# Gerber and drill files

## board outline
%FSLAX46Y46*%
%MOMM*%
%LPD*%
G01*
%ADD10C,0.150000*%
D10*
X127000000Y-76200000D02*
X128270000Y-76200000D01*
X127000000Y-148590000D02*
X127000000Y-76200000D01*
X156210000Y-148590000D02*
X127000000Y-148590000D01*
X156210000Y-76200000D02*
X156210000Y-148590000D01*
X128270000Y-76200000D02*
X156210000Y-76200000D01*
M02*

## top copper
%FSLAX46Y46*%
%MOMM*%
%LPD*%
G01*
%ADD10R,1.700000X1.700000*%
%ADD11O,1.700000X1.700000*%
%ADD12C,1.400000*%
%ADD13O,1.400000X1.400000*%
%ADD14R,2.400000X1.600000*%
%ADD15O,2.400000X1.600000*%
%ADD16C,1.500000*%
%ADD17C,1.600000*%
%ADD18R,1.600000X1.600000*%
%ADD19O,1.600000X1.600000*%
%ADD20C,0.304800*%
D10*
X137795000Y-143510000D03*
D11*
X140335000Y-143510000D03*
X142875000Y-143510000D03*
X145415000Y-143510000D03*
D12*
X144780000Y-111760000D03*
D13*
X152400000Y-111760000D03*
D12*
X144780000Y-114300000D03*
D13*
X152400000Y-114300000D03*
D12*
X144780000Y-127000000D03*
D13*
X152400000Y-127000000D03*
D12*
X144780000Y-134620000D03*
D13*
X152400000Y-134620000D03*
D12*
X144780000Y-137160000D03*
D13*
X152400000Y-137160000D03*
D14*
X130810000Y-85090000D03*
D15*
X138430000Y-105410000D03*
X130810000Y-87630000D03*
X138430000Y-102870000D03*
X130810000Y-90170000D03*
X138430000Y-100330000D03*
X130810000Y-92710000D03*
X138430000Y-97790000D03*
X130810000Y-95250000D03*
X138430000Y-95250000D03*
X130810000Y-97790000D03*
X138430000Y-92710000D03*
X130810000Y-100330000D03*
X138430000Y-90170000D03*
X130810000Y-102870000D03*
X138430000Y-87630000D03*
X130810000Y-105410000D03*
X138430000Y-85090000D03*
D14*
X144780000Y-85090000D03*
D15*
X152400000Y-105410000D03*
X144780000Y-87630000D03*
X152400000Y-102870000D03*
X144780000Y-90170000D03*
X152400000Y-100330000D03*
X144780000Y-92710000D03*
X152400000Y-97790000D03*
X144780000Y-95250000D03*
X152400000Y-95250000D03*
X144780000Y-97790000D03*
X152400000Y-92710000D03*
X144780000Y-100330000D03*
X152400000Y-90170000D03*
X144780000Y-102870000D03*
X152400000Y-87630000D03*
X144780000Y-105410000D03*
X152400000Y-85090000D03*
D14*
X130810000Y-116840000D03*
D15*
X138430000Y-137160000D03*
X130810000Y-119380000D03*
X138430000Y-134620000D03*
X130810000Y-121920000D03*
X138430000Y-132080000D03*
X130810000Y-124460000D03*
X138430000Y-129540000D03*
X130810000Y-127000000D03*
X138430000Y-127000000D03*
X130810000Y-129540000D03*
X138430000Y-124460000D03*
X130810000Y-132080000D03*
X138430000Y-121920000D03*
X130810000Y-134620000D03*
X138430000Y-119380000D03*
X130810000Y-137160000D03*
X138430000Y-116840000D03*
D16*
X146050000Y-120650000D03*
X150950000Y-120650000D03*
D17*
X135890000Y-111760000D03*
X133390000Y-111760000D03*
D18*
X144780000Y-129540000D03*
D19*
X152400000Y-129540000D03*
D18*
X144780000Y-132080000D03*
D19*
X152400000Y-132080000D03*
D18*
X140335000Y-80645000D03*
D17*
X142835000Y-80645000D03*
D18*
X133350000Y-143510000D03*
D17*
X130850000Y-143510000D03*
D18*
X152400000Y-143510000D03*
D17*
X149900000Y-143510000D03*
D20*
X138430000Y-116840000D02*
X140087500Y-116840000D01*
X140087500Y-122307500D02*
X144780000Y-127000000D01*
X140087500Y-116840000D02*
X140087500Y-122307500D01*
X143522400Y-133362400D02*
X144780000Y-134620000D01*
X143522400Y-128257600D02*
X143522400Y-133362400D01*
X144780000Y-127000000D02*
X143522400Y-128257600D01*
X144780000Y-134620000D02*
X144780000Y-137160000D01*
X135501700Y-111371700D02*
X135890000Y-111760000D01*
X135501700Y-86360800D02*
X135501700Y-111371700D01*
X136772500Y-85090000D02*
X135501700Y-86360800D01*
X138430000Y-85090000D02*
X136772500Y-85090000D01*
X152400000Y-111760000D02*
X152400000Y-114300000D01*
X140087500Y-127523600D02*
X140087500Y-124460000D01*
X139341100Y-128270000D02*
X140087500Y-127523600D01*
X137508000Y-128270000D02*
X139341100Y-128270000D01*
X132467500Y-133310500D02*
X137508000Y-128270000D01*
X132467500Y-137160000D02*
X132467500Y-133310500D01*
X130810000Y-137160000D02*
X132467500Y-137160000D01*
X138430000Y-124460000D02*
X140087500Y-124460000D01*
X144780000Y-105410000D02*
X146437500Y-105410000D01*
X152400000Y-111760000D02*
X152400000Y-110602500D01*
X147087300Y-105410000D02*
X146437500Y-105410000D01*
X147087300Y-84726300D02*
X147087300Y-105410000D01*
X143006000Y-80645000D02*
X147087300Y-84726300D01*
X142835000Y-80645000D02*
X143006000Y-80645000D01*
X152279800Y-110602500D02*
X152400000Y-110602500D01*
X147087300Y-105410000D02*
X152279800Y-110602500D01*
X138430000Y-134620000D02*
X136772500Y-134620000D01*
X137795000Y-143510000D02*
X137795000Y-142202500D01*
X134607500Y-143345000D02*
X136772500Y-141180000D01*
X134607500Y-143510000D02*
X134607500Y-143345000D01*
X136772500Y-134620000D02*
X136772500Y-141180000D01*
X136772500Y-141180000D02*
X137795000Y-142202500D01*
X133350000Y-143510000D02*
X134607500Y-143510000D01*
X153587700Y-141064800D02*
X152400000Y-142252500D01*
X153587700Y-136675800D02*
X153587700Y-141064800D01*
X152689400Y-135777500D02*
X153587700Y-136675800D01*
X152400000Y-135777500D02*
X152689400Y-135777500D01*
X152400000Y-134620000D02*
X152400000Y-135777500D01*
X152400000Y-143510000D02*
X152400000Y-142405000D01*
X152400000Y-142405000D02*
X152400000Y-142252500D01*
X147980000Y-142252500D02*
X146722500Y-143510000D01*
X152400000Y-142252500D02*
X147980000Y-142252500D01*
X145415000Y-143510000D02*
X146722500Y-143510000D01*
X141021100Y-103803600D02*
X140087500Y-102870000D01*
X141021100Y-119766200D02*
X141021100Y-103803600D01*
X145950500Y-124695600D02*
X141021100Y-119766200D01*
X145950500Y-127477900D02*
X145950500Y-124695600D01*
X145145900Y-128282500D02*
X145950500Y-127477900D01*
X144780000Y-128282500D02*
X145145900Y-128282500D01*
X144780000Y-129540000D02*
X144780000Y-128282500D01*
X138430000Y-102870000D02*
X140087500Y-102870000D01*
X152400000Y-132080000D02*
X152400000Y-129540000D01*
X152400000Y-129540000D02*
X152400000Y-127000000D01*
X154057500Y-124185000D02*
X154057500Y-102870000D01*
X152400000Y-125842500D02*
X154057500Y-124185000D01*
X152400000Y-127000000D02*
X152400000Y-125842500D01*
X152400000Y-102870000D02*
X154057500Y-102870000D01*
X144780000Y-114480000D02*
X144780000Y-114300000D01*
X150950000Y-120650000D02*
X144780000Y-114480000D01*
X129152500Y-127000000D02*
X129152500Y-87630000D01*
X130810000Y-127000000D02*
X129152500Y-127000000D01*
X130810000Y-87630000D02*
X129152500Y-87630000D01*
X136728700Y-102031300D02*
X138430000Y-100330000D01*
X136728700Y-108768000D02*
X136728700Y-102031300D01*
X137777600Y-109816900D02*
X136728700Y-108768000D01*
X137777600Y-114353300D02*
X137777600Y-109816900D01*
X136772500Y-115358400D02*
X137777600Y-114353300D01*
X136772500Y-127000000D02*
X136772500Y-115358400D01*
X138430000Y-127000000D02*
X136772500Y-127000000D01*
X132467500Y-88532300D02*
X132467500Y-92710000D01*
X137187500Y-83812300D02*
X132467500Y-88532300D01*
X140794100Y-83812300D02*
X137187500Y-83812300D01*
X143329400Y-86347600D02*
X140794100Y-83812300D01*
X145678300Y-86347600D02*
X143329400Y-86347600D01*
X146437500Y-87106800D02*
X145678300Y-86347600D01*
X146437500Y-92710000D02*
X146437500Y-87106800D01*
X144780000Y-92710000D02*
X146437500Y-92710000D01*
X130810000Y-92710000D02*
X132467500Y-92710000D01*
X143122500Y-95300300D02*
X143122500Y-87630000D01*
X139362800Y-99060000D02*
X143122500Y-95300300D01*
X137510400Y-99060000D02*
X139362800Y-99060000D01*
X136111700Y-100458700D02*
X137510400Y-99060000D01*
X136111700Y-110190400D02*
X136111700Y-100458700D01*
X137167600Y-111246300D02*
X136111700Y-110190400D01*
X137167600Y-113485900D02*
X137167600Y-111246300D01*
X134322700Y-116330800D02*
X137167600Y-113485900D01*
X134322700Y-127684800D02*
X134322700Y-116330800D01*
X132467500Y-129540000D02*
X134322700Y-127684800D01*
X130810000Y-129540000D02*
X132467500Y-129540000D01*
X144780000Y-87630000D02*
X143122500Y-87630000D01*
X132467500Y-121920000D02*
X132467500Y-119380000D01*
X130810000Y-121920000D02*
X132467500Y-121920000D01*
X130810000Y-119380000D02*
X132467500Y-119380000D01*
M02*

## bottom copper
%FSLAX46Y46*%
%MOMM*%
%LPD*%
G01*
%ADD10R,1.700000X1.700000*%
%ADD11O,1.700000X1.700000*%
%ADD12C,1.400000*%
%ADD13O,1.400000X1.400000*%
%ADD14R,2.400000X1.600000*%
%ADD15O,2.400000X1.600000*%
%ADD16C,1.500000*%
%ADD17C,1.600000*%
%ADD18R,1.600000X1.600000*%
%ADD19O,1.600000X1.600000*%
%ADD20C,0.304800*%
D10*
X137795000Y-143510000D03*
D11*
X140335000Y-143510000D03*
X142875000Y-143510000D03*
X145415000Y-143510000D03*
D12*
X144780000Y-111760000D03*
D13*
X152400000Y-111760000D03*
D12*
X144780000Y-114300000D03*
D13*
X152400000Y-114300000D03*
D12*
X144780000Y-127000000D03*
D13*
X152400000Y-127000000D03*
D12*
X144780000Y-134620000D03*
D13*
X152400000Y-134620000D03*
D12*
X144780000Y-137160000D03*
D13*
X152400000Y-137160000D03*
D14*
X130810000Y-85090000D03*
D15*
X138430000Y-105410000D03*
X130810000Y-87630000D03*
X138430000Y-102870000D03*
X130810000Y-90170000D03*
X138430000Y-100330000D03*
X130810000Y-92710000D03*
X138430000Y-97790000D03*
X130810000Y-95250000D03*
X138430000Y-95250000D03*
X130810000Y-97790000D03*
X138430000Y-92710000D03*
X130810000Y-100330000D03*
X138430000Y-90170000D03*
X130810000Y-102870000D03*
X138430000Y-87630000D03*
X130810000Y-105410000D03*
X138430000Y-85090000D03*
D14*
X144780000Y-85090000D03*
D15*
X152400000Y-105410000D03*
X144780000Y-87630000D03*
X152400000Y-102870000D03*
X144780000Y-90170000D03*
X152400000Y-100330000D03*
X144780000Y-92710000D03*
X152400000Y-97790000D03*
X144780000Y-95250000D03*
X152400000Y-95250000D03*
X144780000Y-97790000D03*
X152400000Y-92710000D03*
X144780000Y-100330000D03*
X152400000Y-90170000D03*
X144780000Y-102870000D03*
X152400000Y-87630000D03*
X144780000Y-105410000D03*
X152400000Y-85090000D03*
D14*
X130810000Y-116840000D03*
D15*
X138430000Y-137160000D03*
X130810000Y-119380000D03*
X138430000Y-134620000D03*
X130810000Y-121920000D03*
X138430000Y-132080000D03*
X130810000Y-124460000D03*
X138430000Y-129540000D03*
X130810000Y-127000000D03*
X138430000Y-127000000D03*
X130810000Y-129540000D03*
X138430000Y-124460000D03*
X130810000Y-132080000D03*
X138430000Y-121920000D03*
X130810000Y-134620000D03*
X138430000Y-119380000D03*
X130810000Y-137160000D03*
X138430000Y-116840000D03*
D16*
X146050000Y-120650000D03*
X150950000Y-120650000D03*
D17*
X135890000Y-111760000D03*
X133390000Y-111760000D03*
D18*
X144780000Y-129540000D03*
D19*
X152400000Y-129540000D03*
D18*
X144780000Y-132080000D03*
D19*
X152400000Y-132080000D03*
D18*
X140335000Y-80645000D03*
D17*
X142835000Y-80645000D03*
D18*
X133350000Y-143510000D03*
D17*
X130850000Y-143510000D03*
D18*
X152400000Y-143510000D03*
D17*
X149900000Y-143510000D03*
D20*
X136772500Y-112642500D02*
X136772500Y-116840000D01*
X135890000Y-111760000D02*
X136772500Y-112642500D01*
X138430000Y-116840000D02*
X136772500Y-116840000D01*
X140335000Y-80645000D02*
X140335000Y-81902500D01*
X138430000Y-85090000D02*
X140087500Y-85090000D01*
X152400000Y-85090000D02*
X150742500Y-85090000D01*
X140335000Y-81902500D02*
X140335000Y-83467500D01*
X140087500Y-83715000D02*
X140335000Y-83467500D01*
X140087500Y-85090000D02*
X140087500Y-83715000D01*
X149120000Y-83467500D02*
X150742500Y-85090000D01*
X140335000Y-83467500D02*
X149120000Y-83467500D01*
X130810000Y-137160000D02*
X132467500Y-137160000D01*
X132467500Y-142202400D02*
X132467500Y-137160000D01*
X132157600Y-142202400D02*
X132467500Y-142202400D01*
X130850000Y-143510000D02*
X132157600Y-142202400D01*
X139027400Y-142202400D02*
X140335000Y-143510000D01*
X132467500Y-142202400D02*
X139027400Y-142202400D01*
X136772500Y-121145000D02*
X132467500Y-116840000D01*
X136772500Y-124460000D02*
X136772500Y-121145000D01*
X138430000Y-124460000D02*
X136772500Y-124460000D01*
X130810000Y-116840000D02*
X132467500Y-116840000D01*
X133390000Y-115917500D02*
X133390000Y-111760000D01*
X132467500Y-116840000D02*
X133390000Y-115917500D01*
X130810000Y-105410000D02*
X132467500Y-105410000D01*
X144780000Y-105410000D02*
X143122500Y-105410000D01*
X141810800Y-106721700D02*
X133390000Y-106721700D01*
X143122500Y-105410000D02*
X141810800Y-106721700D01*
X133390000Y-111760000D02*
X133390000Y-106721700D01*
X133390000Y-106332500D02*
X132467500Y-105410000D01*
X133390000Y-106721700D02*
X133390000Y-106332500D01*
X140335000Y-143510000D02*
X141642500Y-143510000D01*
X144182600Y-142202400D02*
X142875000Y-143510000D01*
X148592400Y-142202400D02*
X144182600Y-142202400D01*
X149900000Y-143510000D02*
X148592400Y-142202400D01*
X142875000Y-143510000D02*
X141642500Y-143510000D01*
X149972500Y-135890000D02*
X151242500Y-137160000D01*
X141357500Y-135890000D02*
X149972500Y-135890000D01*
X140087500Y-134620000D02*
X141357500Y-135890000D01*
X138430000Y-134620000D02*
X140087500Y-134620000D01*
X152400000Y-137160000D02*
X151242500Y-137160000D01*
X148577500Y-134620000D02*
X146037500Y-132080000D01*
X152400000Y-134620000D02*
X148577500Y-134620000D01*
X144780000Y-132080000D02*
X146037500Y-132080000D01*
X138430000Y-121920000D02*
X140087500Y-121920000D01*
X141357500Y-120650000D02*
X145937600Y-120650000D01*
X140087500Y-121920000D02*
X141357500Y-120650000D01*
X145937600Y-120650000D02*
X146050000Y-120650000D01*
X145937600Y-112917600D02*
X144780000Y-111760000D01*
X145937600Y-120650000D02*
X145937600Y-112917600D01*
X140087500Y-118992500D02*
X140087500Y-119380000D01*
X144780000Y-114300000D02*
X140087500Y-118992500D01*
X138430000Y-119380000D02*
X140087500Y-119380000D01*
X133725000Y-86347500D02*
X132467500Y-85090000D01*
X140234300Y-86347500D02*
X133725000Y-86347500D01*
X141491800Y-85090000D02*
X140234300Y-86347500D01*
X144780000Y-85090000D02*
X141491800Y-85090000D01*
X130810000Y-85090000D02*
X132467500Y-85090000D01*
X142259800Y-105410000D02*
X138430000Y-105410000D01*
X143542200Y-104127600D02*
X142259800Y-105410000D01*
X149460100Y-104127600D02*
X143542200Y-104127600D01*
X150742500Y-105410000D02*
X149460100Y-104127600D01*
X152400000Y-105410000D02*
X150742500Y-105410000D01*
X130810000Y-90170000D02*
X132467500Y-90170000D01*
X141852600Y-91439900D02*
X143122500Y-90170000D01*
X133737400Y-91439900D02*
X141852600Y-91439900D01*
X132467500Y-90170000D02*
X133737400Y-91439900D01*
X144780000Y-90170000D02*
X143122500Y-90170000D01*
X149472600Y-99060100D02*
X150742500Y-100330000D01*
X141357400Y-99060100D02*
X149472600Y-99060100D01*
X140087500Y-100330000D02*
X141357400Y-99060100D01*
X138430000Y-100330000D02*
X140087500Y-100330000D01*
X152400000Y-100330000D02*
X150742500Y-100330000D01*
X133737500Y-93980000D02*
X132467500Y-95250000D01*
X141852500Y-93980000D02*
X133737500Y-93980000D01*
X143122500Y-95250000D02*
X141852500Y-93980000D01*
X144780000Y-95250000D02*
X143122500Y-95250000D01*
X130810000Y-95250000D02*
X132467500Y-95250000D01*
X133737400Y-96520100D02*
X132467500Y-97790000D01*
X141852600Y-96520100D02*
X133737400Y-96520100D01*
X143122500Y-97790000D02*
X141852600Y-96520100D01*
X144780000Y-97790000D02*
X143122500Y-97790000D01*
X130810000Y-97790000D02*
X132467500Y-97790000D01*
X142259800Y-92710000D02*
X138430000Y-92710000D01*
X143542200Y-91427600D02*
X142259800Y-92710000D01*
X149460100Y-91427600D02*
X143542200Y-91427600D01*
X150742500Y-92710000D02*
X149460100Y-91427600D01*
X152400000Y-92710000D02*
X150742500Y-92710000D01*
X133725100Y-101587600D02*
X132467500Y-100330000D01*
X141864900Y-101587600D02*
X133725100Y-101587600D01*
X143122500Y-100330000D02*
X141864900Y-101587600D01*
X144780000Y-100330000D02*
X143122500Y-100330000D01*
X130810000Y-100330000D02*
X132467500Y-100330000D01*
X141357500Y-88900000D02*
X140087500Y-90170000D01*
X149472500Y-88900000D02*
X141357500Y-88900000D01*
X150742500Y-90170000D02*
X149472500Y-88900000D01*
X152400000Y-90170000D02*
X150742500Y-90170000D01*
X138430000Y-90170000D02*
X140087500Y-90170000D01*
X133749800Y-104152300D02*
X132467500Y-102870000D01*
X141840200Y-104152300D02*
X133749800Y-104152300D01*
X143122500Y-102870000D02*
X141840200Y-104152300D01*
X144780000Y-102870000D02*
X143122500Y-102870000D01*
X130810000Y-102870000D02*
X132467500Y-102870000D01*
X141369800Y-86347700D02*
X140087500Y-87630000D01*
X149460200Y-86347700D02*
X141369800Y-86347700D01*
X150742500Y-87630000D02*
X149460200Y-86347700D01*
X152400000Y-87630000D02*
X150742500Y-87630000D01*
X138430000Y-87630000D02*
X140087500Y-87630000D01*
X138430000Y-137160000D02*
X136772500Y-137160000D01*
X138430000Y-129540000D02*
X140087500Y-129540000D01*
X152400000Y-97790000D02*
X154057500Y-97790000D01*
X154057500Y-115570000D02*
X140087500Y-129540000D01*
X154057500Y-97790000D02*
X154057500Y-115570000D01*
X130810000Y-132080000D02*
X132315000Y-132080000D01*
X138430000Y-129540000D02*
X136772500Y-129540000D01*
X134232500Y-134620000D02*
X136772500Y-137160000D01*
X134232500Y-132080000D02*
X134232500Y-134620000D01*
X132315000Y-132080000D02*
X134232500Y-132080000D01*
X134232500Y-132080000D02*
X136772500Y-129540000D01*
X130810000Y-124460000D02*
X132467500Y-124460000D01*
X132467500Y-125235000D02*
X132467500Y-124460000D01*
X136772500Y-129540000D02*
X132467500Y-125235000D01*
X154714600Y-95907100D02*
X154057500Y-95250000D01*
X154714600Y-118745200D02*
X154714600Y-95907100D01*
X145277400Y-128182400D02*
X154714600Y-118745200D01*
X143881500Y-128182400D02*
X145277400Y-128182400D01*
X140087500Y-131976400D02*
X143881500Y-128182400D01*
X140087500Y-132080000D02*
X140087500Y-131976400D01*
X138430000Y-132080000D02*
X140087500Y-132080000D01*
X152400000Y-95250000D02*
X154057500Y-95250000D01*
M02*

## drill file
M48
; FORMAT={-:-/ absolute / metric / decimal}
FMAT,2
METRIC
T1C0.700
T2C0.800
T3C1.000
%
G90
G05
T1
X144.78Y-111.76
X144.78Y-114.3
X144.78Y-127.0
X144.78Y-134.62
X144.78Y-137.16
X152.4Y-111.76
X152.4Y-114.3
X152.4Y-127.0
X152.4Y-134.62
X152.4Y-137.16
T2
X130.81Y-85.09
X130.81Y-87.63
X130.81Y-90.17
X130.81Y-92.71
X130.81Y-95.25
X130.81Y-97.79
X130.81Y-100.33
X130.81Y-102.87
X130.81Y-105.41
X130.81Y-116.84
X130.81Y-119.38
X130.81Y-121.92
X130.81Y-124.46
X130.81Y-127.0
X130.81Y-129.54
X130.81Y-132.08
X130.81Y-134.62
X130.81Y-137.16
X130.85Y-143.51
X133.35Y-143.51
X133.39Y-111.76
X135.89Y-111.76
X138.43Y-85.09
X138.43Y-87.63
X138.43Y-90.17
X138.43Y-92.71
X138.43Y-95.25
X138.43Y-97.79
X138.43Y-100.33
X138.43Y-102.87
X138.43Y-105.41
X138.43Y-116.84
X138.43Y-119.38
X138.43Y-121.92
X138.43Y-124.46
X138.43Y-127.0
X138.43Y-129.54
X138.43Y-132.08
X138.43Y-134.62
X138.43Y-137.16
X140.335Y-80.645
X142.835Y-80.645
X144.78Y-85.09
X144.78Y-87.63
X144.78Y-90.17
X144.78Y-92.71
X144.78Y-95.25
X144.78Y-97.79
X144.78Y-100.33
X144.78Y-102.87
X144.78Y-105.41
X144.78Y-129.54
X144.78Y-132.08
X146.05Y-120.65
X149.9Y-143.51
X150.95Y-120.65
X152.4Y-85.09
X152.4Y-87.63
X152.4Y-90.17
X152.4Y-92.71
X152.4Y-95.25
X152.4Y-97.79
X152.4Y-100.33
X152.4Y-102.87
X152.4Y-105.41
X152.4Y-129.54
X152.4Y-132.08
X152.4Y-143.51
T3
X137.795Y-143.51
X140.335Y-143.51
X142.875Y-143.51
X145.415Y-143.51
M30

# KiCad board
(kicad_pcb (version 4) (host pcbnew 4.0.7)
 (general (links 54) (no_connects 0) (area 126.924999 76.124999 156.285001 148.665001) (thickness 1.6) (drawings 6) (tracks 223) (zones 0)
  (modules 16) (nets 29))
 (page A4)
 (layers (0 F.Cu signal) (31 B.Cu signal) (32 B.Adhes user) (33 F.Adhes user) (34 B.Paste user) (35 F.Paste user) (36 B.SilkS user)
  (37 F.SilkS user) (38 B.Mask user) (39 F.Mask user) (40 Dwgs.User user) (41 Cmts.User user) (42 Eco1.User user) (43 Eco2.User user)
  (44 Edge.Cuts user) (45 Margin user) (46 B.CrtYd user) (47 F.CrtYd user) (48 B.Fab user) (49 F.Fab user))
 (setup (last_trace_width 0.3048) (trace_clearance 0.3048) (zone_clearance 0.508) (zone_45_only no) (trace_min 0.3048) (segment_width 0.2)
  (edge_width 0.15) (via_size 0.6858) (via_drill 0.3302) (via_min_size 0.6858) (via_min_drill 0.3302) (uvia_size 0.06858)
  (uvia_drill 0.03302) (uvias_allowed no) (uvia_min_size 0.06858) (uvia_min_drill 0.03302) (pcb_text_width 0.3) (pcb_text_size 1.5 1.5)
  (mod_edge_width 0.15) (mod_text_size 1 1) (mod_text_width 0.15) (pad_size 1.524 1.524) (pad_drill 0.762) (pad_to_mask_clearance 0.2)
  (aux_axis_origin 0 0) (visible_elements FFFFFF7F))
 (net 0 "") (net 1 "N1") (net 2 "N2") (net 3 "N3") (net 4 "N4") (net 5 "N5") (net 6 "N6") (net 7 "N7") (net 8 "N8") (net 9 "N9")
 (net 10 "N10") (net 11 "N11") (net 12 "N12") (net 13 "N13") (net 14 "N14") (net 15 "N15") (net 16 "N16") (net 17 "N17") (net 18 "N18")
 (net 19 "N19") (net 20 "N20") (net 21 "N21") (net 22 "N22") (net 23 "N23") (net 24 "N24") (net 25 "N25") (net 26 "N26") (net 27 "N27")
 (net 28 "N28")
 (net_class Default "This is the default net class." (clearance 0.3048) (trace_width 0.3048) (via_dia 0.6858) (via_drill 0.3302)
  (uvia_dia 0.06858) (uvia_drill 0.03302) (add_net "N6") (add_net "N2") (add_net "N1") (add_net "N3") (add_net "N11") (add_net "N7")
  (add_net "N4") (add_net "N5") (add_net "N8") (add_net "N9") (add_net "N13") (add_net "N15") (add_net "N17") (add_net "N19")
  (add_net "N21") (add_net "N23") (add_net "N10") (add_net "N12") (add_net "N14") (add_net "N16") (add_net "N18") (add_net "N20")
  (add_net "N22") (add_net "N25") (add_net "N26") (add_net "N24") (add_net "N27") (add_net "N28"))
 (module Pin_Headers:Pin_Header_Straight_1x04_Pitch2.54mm (layer F.Cu) (at 137.795 143.51 90)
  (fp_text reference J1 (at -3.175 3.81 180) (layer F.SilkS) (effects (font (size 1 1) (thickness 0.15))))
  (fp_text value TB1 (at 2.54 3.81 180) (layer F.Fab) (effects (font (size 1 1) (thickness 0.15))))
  (pad 1 thru_hole rect (at 0 0 90) (size 1.7 1.7) (drill 1) (layers *.Cu *.Mask) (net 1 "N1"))
  (pad 2 thru_hole oval (at 0 2.54 90) (size 1.7 1.7) (drill 1) (layers *.Cu *.Mask) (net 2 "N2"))
  (pad 3 thru_hole oval (at 0 5.08 90) (size 1.7 1.7) (drill 1) (layers *.Cu *.Mask) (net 2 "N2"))
  (pad 4 thru_hole oval (at 0 7.62 90) (size 1.7 1.7) (drill 1) (layers *.Cu *.Mask) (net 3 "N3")))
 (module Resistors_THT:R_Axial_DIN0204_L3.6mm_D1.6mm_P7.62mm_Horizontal (layer F.Cu) (at 144.78 111.76)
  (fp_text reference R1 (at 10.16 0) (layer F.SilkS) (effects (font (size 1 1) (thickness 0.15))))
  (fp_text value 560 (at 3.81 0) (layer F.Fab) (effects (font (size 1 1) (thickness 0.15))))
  (pad 1 thru_hole circle (at 0 0) (size 1.4 1.4) (drill 0.7) (layers *.Cu *.Mask) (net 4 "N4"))
  (pad 2 thru_hole oval (at 7.62 0) (size 1.4 1.4) (drill 0.7) (layers *.Cu *.Mask) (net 2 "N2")))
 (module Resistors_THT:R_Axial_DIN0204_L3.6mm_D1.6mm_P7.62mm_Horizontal (layer F.Cu) (at 144.78 114.3)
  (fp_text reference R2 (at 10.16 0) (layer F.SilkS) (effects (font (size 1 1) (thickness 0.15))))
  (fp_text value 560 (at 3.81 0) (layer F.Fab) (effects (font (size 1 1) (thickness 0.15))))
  (pad 1 thru_hole circle (at 0 0) (size 1.4 1.4) (drill 0.7) (layers *.Cu *.Mask) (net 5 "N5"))
  (pad 2 thru_hole oval (at 7.62 0) (size 1.4 1.4) (drill 0.7) (layers *.Cu *.Mask) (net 2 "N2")))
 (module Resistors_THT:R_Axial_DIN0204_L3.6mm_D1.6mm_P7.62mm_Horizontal (layer F.Cu) (at 144.78 127)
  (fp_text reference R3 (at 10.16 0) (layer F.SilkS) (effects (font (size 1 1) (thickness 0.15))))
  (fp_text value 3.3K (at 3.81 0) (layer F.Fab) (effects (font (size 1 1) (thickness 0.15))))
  (pad 1 thru_hole circle (at 0 0) (size 1.4 1.4) (drill 0.7) (layers *.Cu *.Mask) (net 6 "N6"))
  (pad 2 thru_hole oval (at 7.62 0) (size 1.4 1.4) (drill 0.7) (layers *.Cu *.Mask) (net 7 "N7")))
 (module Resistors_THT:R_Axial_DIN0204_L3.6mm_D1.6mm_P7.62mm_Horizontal (layer F.Cu) (at 144.78 134.62)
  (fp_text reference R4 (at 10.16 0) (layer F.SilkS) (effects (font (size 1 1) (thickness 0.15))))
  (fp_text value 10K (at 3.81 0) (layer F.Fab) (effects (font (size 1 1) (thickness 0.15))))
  (pad 1 thru_hole circle (at 0 0) (size 1.4 1.4) (drill 0.7) (layers *.Cu *.Mask) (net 6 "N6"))
  (pad 2 thru_hole oval (at 7.62 0) (size 1.4 1.4) (drill 0.7) (layers *.Cu *.Mask) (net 3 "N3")))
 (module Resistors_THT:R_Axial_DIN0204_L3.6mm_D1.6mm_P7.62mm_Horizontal (layer F.Cu) (at 144.78 137.16)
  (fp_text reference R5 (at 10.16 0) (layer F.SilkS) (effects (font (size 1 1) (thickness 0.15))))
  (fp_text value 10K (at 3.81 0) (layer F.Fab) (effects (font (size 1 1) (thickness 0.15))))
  (pad 1 thru_hole circle (at 0 0) (size 1.4 1.4) (drill 0.7) (layers *.Cu *.Mask) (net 6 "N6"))
  (pad 2 thru_hole oval (at 7.62 0) (size 1.4 1.4) (drill 0.7) (layers *.Cu *.Mask) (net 1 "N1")))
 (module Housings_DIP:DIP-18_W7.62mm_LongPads (layer F.Cu) (at 130.81 85.09)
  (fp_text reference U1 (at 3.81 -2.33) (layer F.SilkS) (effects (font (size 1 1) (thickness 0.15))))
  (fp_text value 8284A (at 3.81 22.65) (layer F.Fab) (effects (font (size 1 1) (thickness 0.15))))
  (pad 1 thru_hole rect (at 0 0) (size 2.4 1.6) (drill 0.8) (layers *.Cu *.Mask) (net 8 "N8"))
  (pad 10 thru_hole oval (at 7.62 20.32) (size 2.4 1.6) (drill 0.8) (layers *.Cu *.Mask) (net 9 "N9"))
  (pad 2 thru_hole oval (at 0 2.54) (size 2.4 1.6) (drill 0.8) (layers *.Cu *.Mask) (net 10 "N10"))
  (pad 11 thru_hole oval (at 7.62 17.78) (size 2.4 1.6) (drill 0.8) (layers *.Cu *.Mask) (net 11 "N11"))
  (pad 3 thru_hole oval (at 0 5.08) (size 2.4 1.6) (drill 0.8) (layers *.Cu *.Mask) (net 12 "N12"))
  (pad 12 thru_hole oval (at 7.62 15.24) (size 2.4 1.6) (drill 0.8) (layers *.Cu *.Mask) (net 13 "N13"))
  (pad 4 thru_hole oval (at 0 7.62) (size 2.4 1.6) (drill 0.8) (layers *.Cu *.Mask) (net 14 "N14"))
  (pad 13 thru_hole oval (at 7.62 12.7) (size 2.4 1.6) (drill 0.8) (layers *.Cu *.Mask) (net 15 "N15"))
  (pad 5 thru_hole oval (at 0 10.16) (size 2.4 1.6) (drill 0.8) (layers *.Cu *.Mask) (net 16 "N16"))
  (pad 14 thru_hole oval (at 7.62 10.16) (size 2.4 1.6) (drill 0.8) (layers *.Cu *.Mask) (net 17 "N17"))
  (pad 6 thru_hole oval (at 0 12.7) (size 2.4 1.6) (drill 0.8) (layers *.Cu *.Mask) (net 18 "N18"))
  (pad 15 thru_hole oval (at 7.62 7.62) (size 2.4 1.6) (drill 0.8) (layers *.Cu *.Mask) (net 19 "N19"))
  (pad 7 thru_hole oval (at 0 15.24) (size 2.4 1.6) (drill 0.8) (layers *.Cu *.Mask) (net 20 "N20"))
  (pad 16 thru_hole oval (at 7.62 5.08) (size 2.4 1.6) (drill 0.8) (layers *.Cu *.Mask) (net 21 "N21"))
  (pad 8 thru_hole oval (at 0 17.78) (size 2.4 1.6) (drill 0.8) (layers *.Cu *.Mask) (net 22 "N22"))
  (pad 17 thru_hole oval (at 7.62 2.54) (size 2.4 1.6) (drill 0.8) (layers *.Cu *.Mask) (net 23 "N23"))
  (pad 9 thru_hole oval (at 0 20.32) (size 2.4 1.6) (drill 0.8) (layers *.Cu *.Mask) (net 2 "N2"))
  (pad 18 thru_hole oval (at 7.62 0) (size 2.4 1.6) (drill 0.8) (layers *.Cu *.Mask) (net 6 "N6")))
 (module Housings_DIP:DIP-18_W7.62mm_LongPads (layer F.Cu) (at 144.78 85.09)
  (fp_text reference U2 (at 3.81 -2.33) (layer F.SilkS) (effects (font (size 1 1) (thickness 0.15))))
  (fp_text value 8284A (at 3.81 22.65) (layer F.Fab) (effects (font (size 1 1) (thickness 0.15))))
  (pad 1 thru_hole rect (at 0 0) (size 2.4 1.6) (drill 0.8) (layers *.Cu *.Mask) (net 8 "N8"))
  (pad 10 thru_hole oval (at 7.62 20.32) (size 2.4 1.6) (drill 0.8) (layers *.Cu *.Mask) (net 9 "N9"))
  (pad 2 thru_hole oval (at 0 2.54) (size 2.4 1.6) (drill 0.8) (layers *.Cu *.Mask) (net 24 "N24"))
  (pad 11 thru_hole oval (at 7.62 17.78) (size 2.4 1.6) (drill 0.8) (layers *.Cu *.Mask) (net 7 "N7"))
  (pad 3 thru_hole oval (at 0 5.08) (size 2.4 1.6) (drill 0.8) (layers *.Cu *.Mask) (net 12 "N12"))
  (pad 12 thru_hole oval (at 7.62 15.24) (size 2.4 1.6) (drill 0.8) (layers *.Cu *.Mask) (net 13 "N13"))
  (pad 4 thru_hole oval (at 0 7.62) (size 2.4 1.6) (drill 0.8) (layers *.Cu *.Mask) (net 14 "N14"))
  (pad 13 thru_hole oval (at 7.62 12.7) (size 2.4 1.6) (drill 0.8) (layers *.Cu *.Mask) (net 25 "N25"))
  (pad 5 thru_hole oval (at 0 10.16) (size 2.4 1.6) (drill 0.8) (layers *.Cu *.Mask) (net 16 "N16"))
  (pad 14 thru_hole oval (at 7.62 10.16) (size 2.4 1.6) (drill 0.8) (layers *.Cu *.Mask) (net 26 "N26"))
  (pad 6 thru_hole oval (at 0 12.7) (size 2.4 1.6) (drill 0.8) (layers *.Cu *.Mask) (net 18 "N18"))
  (pad 15 thru_hole oval (at 7.62 7.62) (size 2.4 1.6) (drill 0.8) (layers *.Cu *.Mask) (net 19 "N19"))
  (pad 7 thru_hole oval (at 0 15.24) (size 2.4 1.6) (drill 0.8) (layers *.Cu *.Mask) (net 20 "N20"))
  (pad 16 thru_hole oval (at 7.62 5.08) (size 2.4 1.6) (drill 0.8) (layers *.Cu *.Mask) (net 21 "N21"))
  (pad 8 thru_hole oval (at 0 17.78) (size 2.4 1.6) (drill 0.8) (layers *.Cu *.Mask) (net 22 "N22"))
  (pad 17 thru_hole oval (at 7.62 2.54) (size 2.4 1.6) (drill 0.8) (layers *.Cu *.Mask) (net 23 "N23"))
  (pad 9 thru_hole oval (at 0 20.32) (size 2.4 1.6) (drill 0.8) (layers *.Cu *.Mask) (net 2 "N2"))
  (pad 18 thru_hole oval (at 7.62 0) (size 2.4 1.6) (drill 0.8) (layers *.Cu *.Mask) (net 6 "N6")))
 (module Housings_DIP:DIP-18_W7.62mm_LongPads (layer F.Cu) (at 130.81 116.84)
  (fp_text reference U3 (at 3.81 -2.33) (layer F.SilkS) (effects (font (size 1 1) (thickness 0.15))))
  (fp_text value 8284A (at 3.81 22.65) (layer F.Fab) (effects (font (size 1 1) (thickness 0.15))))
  (pad 1 thru_hole rect (at 0 0) (size 2.4 1.6) (drill 0.8) (layers *.Cu *.Mask) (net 2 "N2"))
  (pad 10 thru_hole oval (at 7.62 20.32) (size 2.4 1.6) (drill 0.8) (layers *.Cu *.Mask) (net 25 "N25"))
  (pad 2 thru_hole oval (at 0 2.54) (size 2.4 1.6) (drill 0.8) (layers *.Cu *.Mask) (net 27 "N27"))
  (pad 11 thru_hole oval (at 7.62 17.78) (size 2.4 1.6) (drill 0.8) (layers *.Cu *.Mask) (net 1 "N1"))
  (pad 3 thru_hole oval (at 0 5.08) (size 2.4 1.6) (drill 0.8) (layers *.Cu *.Mask) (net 27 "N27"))
  (pad 12 thru_hole oval (at 7.62 15.24) (size 2.4 1.6) (drill 0.8) (layers *.Cu *.Mask) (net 26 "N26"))
  (pad 4 thru_hole oval (at 0 7.62) (size 2.4 1.6) (drill 0.8) (layers *.Cu *.Mask) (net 25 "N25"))
  (pad 13 thru_hole oval (at 7.62 12.7) (size 2.4 1.6) (drill 0.8) (layers *.Cu *.Mask) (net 25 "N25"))
  (pad 5 thru_hole oval (at 0 10.16) (size 2.4 1.6) (drill 0.8) (layers *.Cu *.Mask) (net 10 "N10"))
  (pad 14 thru_hole oval (at 7.62 10.16) (size 2.4 1.6) (drill 0.8) (layers *.Cu *.Mask) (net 13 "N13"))
  (pad 6 thru_hole oval (at 0 12.7) (size 2.4 1.6) (drill 0.8) (layers *.Cu *.Mask) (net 24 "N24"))
  (pad 15 thru_hole oval (at 7.62 7.62) (size 2.4 1.6) (drill 0.8) (layers *.Cu *.Mask) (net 2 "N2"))
  (pad 7 thru_hole oval (at 0 15.24) (size 2.4 1.6) (drill 0.8) (layers *.Cu *.Mask) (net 25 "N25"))
  (pad 16 thru_hole oval (at 7.62 5.08) (size 2.4 1.6) (drill 0.8) (layers *.Cu *.Mask) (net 4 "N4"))
  (pad 8 thru_hole oval (at 0 17.78) (size 2.4 1.6) (drill 0.8) (layers *.Cu *.Mask) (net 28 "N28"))
  (pad 17 thru_hole oval (at 7.62 2.54) (size 2.4 1.6) (drill 0.8) (layers *.Cu *.Mask) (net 5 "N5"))
  (pad 9 thru_hole oval (at 0 20.32) (size 2.4 1.6) (drill 0.8) (layers *.Cu *.Mask) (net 2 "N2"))
  (pad 18 thru_hole oval (at 7.62 0) (size 2.4 1.6) (drill 0.8) (layers *.Cu *.Mask) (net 6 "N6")))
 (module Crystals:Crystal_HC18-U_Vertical (layer F.Cu) (at 146.05 120.65)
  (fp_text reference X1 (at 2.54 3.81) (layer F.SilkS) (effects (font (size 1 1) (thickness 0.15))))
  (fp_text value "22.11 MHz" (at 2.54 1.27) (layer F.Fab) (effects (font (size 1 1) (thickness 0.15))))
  (pad 1 thru_hole circle (at 0 0) (size 1.5 1.5) (drill 0.8) (layers *.Cu *.Mask) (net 4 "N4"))
  (pad 2 thru_hole circle (at 4.9 0) (size 1.5 1.5) (drill 0.8) (layers *.Cu *.Mask) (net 5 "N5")))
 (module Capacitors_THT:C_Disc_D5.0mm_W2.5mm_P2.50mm (layer F.Cu) (at 135.89 111.76 180)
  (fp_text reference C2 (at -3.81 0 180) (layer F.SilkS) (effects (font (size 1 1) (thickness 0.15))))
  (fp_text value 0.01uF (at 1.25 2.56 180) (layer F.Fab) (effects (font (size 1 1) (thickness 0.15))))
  (pad 1 thru_hole circle (at 0 0 180) (size 1.6 1.6) (drill 0.8) (layers *.Cu *.Mask) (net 6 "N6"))
  (pad 2 thru_hole circle (at 2.5 0 180) (size 1.6 1.6) (drill 0.8) (layers *.Cu *.Mask) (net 2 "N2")))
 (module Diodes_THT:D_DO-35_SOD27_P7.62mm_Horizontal (layer F.Cu) (at 144.78 129.54)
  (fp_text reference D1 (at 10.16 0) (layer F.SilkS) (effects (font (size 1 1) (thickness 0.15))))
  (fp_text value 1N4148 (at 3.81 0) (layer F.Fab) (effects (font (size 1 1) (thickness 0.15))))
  (pad 1 thru_hole rect (at 0 0) (size 1.6 1.6) (drill 0.8) (layers *.Cu *.Mask) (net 11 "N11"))
  (pad 2 thru_hole oval (at 7.62 0) (size 1.6 1.6) (drill 0.8) (layers *.Cu *.Mask) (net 7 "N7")))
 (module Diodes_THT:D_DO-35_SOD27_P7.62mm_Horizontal (layer F.Cu) (at 144.78 132.08)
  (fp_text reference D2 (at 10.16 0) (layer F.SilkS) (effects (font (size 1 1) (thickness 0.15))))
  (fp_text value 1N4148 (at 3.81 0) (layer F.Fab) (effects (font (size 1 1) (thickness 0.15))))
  (pad 1 thru_hole rect (at 0 0) (size 1.6 1.6) (drill 0.8) (layers *.Cu *.Mask) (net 3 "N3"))
  (pad 2 thru_hole oval (at 7.62 0) (size 1.6 1.6) (drill 0.8) (layers *.Cu *.Mask) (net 7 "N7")))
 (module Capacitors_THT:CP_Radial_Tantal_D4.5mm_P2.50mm (layer F.Cu) (at 140.335 80.645)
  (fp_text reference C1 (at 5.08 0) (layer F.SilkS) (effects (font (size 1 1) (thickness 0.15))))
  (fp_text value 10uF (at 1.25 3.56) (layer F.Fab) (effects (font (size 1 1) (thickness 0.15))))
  (pad 1 thru_hole rect (at 0 0) (size 1.6 1.6) (drill 0.8) (layers *.Cu *.Mask) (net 6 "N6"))
  (pad 2 thru_hole circle (at 2.5 0) (size 1.6 1.6) (drill 0.8) (layers *.Cu *.Mask) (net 2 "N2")))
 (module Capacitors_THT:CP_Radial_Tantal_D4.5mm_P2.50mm (layer F.Cu) (at 133.35 143.51 180)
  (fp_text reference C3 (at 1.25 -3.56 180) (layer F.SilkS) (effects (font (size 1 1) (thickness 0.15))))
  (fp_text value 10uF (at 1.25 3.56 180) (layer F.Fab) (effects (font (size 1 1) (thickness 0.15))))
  (pad 1 thru_hole rect (at 0 0 180) (size 1.6 1.6) (drill 0.8) (layers *.Cu *.Mask) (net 1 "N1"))
  (pad 2 thru_hole circle (at 2.5 0 180) (size 1.6 1.6) (drill 0.8) (layers *.Cu *.Mask) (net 2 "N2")))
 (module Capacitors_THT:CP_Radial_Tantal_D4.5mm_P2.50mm (layer F.Cu) (at 152.4 143.51 180)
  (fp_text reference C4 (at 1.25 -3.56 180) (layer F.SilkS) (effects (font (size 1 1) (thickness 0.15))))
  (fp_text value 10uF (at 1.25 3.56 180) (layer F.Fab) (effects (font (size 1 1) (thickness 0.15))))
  (pad 1 thru_hole rect (at 0 0 180) (size 1.6 1.6) (drill 0.8) (layers *.Cu *.Mask) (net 3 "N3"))
  (pad 2 thru_hole circle (at 2.5 0 180) (size 1.6 1.6) (drill 0.8) (layers *.Cu *.Mask) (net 2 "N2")))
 (gr_line (start 127 76.2) (end 128.27 76.2) (angle 90) (layer Edge.Cuts) (width 0.15))
 (gr_line (start 127 148.59) (end 127 76.2) (angle 90) (layer Edge.Cuts) (width 0.15))
 (gr_line (start 156.21 148.59) (end 127 148.59) (angle 90) (layer Edge.Cuts) (width 0.15))
 (gr_line (start 156.21 76.2) (end 156.21 148.59) (angle 90) (layer Edge.Cuts) (width 0.15))
 (gr_line (start 128.27 76.2) (end 156.21 76.2) (angle 90) (layer Edge.Cuts) (width 0.15))
 (segment (start 136.7725 112.6425) (end 136.7725 116.84) (width 0.3048) (layer B.Cu) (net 6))
 (segment (start 135.89 111.76) (end 136.7725 112.6425) (width 0.3048) (layer B.Cu) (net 6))
 (segment (start 138.43 116.84) (end 136.7725 116.84) (width 0.3048) (layer B.Cu) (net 6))
 (segment (start 138.43 116.84) (end 140.0875 116.84) (width 0.3048) (layer F.Cu) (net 6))
 (segment (start 140.0875 122.3075) (end 144.78 127) (width 0.3048) (layer F.Cu) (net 6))
 (segment (start 140.0875 116.84) (end 140.0875 122.3075) (width 0.3048) (layer F.Cu) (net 6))
 (segment (start 143.5224 133.3624) (end 144.78 134.62) (width 0.3048) (layer F.Cu) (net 6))
 (segment (start 143.5224 128.2576) (end 143.5224 133.3624) (width 0.3048) (layer F.Cu) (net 6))
 (segment (start 144.78 127) (end 143.5224 128.2576) (width 0.3048) (layer F.Cu) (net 6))
 (segment (start 144.78 134.62) (end 144.78 137.16) (width 0.3048) (layer F.Cu) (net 6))
 (segment (start 140.335 80.645) (end 140.335 81.9025) (width 0.3048) (layer B.Cu) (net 6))
 (segment (start 138.43 85.09) (end 140.0875 85.09) (width 0.3048) (layer B.Cu) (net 6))
 (segment (start 152.4 85.09) (end 150.7425 85.09) (width 0.3048) (layer B.Cu) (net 6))
 (segment (start 140.335 81.9025) (end 140.335 83.4675) (width 0.3048) (layer B.Cu) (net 6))
 (segment (start 140.0875 83.715) (end 140.335 83.4675) (width 0.3048) (layer B.Cu) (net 6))
 (segment (start 140.0875 85.09) (end 140.0875 83.715) (width 0.3048) (layer B.Cu) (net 6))
 (segment (start 149.12 83.4675) (end 150.7425 85.09) (width 0.3048) (layer B.Cu) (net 6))
 (segment (start 140.335 83.4675) (end 149.12 83.4675) (width 0.3048) (layer B.Cu) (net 6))
 (segment (start 135.5017 111.3717) (end 135.89 111.76) (width 0.3048) (layer F.Cu) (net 6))
 (segment (start 135.5017 86.3608) (end 135.5017 111.3717) (width 0.3048) (layer F.Cu) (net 6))
 (segment (start 136.7725 85.09) (end 135.5017 86.3608) (width 0.3048) (layer F.Cu) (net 6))
 (segment (start 138.43 85.09) (end 136.7725 85.09) (width 0.3048) (layer F.Cu) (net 6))
 (segment (start 130.81 137.16) (end 132.4675 137.16) (width 0.3048) (layer B.Cu) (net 2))
 (segment (start 132.4675 142.2024) (end 132.4675 137.16) (width 0.3048) (layer B.Cu) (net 2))
 (segment (start 132.1576 142.2024) (end 132.4675 142.2024) (width 0.3048) (layer B.Cu) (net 2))
 (segment (start 130.85 143.51) (end 132.1576 142.2024) (width 0.3048) (layer B.Cu) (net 2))
 (segment (start 139.0274 142.2024) (end 140.335 143.51) (width 0.3048) (layer B.Cu) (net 2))
 (segment (start 132.4675 142.2024) (end 139.0274 142.2024) (width 0.3048) (layer B.Cu) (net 2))
 (segment (start 136.7725 121.145) (end 132.4675 116.84) (width 0.3048) (layer B.Cu) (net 2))
 (segment (start 136.7725 124.46) (end 136.7725 121.145) (width 0.3048) (layer B.Cu) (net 2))
 (segment (start 138.43 124.46) (end 136.7725 124.46) (width 0.3048) (layer B.Cu) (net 2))
 (segment (start 130.81 116.84) (end 132.4675 116.84) (width 0.3048) (layer B.Cu) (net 2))
 (segment (start 152.4 111.76) (end 152.4 114.3) (width 0.3048) (layer F.Cu) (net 2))
 (segment (start 140.0875 127.5236) (end 140.0875 124.46) (width 0.3048) (layer F.Cu) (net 2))
 (segment (start 139.3411 128.27) (end 140.0875 127.5236) (width 0.3048) (layer F.Cu) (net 2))
 (segment (start 137.508 128.27) (end 139.3411 128.27) (width 0.3048) (layer F.Cu) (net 2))
 (segment (start 132.4675 133.3105) (end 137.508 128.27) (width 0.3048) (layer F.Cu) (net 2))
 (segment (start 132.4675 137.16) (end 132.4675 133.3105) (width 0.3048) (layer F.Cu) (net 2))
 (segment (start 130.81 137.16) (end 132.4675 137.16) (width 0.3048) (layer F.Cu) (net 2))
 (segment (start 138.43 124.46) (end 140.0875 124.46) (width 0.3048) (layer F.Cu) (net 2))
 (segment (start 133.39 115.9175) (end 133.39 111.76) (width 0.3048) (layer B.Cu) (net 2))
 (segment (start 132.4675 116.84) (end 133.39 115.9175) (width 0.3048) (layer B.Cu) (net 2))
 (segment (start 130.81 105.41) (end 132.4675 105.41) (width 0.3048) (layer B.Cu) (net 2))
 (segment (start 144.78 105.41) (end 143.1225 105.41) (width 0.3048) (layer B.Cu) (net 2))
 (segment (start 141.8108 106.7217) (end 133.39 106.7217) (width 0.3048) (layer B.Cu) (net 2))
 (segment (start 143.1225 105.41) (end 141.8108 106.7217) (width 0.3048) (layer B.Cu) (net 2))
 (segment (start 133.39 111.76) (end 133.39 106.7217) (width 0.3048) (layer B.Cu) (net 2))
 (segment (start 133.39 106.3325) (end 132.4675 105.41) (width 0.3048) (layer B.Cu) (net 2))
 (segment (start 133.39 106.7217) (end 133.39 106.3325) (width 0.3048) (layer B.Cu) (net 2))
 (segment (start 144.78 105.41) (end 146.4375 105.41) (width 0.3048) (layer F.Cu) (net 2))
 (segment (start 152.4 111.76) (end 152.4 110.6025) (width 0.3048) (layer F.Cu) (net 2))
 (segment (start 147.0873 105.41) (end 146.4375 105.41) (width 0.3048) (layer F.Cu) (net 2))
 (segment (start 147.0873 84.7263) (end 147.0873 105.41) (width 0.3048) (layer F.Cu) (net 2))
 (segment (start 143.006 80.645) (end 147.0873 84.7263) (width 0.3048) (layer F.Cu) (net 2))
 (segment (start 142.835 80.645) (end 143.006 80.645) (width 0.3048) (layer F.Cu) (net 2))
 (segment (start 152.2798 110.6025) (end 152.4 110.6025) (width 0.3048) (layer F.Cu) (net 2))
 (segment (start 147.0873 105.41) (end 152.2798 110.6025) (width 0.3048) (layer F.Cu) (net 2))
 (segment (start 140.335 143.51) (end 141.6425 143.51) (width 0.3048) (layer B.Cu) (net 2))
 (segment (start 144.1826 142.2024) (end 142.875 143.51) (width 0.3048) (layer B.Cu) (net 2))
 (segment (start 148.5924 142.2024) (end 144.1826 142.2024) (width 0.3048) (layer B.Cu) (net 2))
 (segment (start 149.9 143.51) (end 148.5924 142.2024) (width 0.3048) (layer B.Cu) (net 2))
 (segment (start 142.875 143.51) (end 141.6425 143.51) (width 0.3048) (layer B.Cu) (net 2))
 (segment (start 138.43 134.62) (end 136.7725 134.62) (width 0.3048) (layer F.Cu) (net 1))
 (segment (start 137.795 143.51) (end 137.795 142.2025) (width 0.3048) (layer F.Cu) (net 1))
 (segment (start 134.6075 143.345) (end 136.7725 141.18) (width 0.3048) (layer F.Cu) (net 1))
 (segment (start 134.6075 143.51) (end 134.6075 143.345) (width 0.3048) (layer F.Cu) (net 1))
 (segment (start 136.7725 134.62) (end 136.7725 141.18) (width 0.3048) (layer F.Cu) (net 1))
 (segment (start 136.7725 141.18) (end 137.795 142.2025) (width 0.3048) (layer F.Cu) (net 1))
 (segment (start 133.35 143.51) (end 134.6075 143.51) (width 0.3048) (layer F.Cu) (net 1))
 (segment (start 149.9725 135.89) (end 151.2425 137.16) (width 0.3048) (layer B.Cu) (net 1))
 (segment (start 141.3575 135.89) (end 149.9725 135.89) (width 0.3048) (layer B.Cu) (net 1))
 (segment (start 140.0875 134.62) (end 141.3575 135.89) (width 0.3048) (layer B.Cu) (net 1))
 (segment (start 138.43 134.62) (end 140.0875 134.62) (width 0.3048) (layer B.Cu) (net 1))
 (segment (start 152.4 137.16) (end 151.2425 137.16) (width 0.3048) (layer B.Cu) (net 1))
 (segment (start 153.5877 141.0648) (end 152.4 142.2525) (width 0.3048) (layer F.Cu) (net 3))
 (segment (start 153.5877 136.6758) (end 153.5877 141.0648) (width 0.3048) (layer F.Cu) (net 3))
 (segment (start 152.6894 135.7775) (end 153.5877 136.6758) (width 0.3048) (layer F.Cu) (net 3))
 (segment (start 152.4 135.7775) (end 152.6894 135.7775) (width 0.3048) (layer F.Cu) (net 3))
 (segment (start 152.4 134.62) (end 152.4 135.7775) (width 0.3048) (layer F.Cu) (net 3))
 (segment (start 152.4 143.51) (end 152.4 142.405) (width 0.3048) (layer F.Cu) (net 3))
 (segment (start 152.4 142.405) (end 152.4 142.2525) (width 0.3048) (layer F.Cu) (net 3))
 (segment (start 147.98 142.2525) (end 146.7225 143.51) (width 0.3048) (layer F.Cu) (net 3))
 (segment (start 152.4 142.2525) (end 147.98 142.2525) (width 0.3048) (layer F.Cu) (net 3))
 (segment (start 145.415 143.51) (end 146.7225 143.51) (width 0.3048) (layer F.Cu) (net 3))
 (segment (start 148.5775 134.62) (end 146.0375 132.08) (width 0.3048) (layer B.Cu) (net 3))
 (segment (start 152.4 134.62) (end 148.5775 134.62) (width 0.3048) (layer B.Cu) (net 3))
 (segment (start 144.78 132.08) (end 146.0375 132.08) (width 0.3048) (layer B.Cu) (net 3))
 (segment (start 141.0211 103.8036) (end 140.0875 102.87) (width 0.3048) (layer F.Cu) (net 11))
 (segment (start 141.0211 119.7662) (end 141.0211 103.8036) (width 0.3048) (layer F.Cu) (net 11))
 (segment (start 145.9505 124.6956) (end 141.0211 119.7662) (width 0.3048) (layer F.Cu) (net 11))
 (segment (start 145.9505 127.4779) (end 145.9505 124.6956) (width 0.3048) (layer F.Cu) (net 11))
 (segment (start 145.1459 128.2825) (end 145.9505 127.4779) (width 0.3048) (layer F.Cu) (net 11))
 (segment (start 144.78 128.2825) (end 145.1459 128.2825) (width 0.3048) (layer F.Cu) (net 11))
 (segment (start 144.78 129.54) (end 144.78 128.2825) (width 0.3048) (layer F.Cu) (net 11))
 (segment (start 138.43 102.87) (end 140.0875 102.87) (width 0.3048) (layer F.Cu) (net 11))
 (segment (start 152.4 132.08) (end 152.4 129.54) (width 0.3048) (layer F.Cu) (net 7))
 (segment (start 152.4 129.54) (end 152.4 127) (width 0.3048) (layer F.Cu) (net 7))
 (segment (start 154.0575 124.185) (end 154.0575 102.87) (width 0.3048) (layer F.Cu) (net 7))
 (segment (start 152.4 125.8425) (end 154.0575 124.185) (width 0.3048) (layer F.Cu) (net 7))
 (segment (start 152.4 127) (end 152.4 125.8425) (width 0.3048) (layer F.Cu) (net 7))
 (segment (start 152.4 102.87) (end 154.0575 102.87) (width 0.3048) (layer F.Cu) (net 7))
 (segment (start 138.43 121.92) (end 140.0875 121.92) (width 0.3048) (layer B.Cu) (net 4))
 (segment (start 141.3575 120.65) (end 145.9376 120.65) (width 0.3048) (layer B.Cu) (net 4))
 (segment (start 140.0875 121.92) (end 141.3575 120.65) (width 0.3048) (layer B.Cu) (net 4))
 (segment (start 145.9376 120.65) (end 146.05 120.65) (width 0.3048) (layer B.Cu) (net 4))
 (segment (start 145.9376 112.9176) (end 144.78 111.76) (width 0.3048) (layer B.Cu) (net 4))
 (segment (start 145.9376 120.65) (end 145.9376 112.9176) (width 0.3048) (layer B.Cu) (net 4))
 (segment (start 144.78 114.48) (end 144.78 114.3) (width 0.3048) (layer F.Cu) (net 5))
 (segment (start 150.95 120.65) (end 144.78 114.48) (width 0.3048) (layer F.Cu) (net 5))
 (segment (start 140.0875 118.9925) (end 140.0875 119.38) (width 0.3048) (layer B.Cu) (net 5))
 (segment (start 144.78 114.3) (end 140.0875 118.9925) (width 0.3048) (layer B.Cu) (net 5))
 (segment (start 138.43 119.38) (end 140.0875 119.38) (width 0.3048) (layer B.Cu) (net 5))
 (segment (start 133.725 86.3475) (end 132.4675 85.09) (width 0.3048) (layer B.Cu) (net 8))
 (segment (start 140.2343 86.3475) (end 133.725 86.3475) (width 0.3048) (layer B.Cu) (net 8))
 (segment (start 141.4918 85.09) (end 140.2343 86.3475) (width 0.3048) (layer B.Cu) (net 8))
 (segment (start 144.78 85.09) (end 141.4918 85.09) (width 0.3048) (layer B.Cu) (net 8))
 (segment (start 130.81 85.09) (end 132.4675 85.09) (width 0.3048) (layer B.Cu) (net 8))
 (segment (start 142.2598 105.41) (end 138.43 105.41) (width 0.3048) (layer B.Cu) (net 9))
 (segment (start 143.5422 104.1276) (end 142.2598 105.41) (width 0.3048) (layer B.Cu) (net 9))
 (segment (start 149.4601 104.1276) (end 143.5422 104.1276) (width 0.3048) (layer B.Cu) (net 9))
 (segment (start 150.7425 105.41) (end 149.4601 104.1276) (width 0.3048) (layer B.Cu) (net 9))
 (segment (start 152.4 105.41) (end 150.7425 105.41) (width 0.3048) (layer B.Cu) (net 9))
 (segment (start 129.1525 127) (end 129.1525 87.63) (width 0.3048) (layer F.Cu) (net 10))
 (segment (start 130.81 127) (end 129.1525 127) (width 0.3048) (layer F.Cu) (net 10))
 (segment (start 130.81 87.63) (end 129.1525 87.63) (width 0.3048) (layer F.Cu) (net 10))
 (segment (start 130.81 90.17) (end 132.4675 90.17) (width 0.3048) (layer B.Cu) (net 12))
 (segment (start 141.8526 91.4399) (end 143.1225 90.17) (width 0.3048) (layer B.Cu) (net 12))
 (segment (start 133.7374 91.4399) (end 141.8526 91.4399) (width 0.3048) (layer B.Cu) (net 12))
 (segment (start 132.4675 90.17) (end 133.7374 91.4399) (width 0.3048) (layer B.Cu) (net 12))
 (segment (start 144.78 90.17) (end 143.1225 90.17) (width 0.3048) (layer B.Cu) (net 12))
 (segment (start 149.4726 99.0601) (end 150.7425 100.33) (width 0.3048) (layer B.Cu) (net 13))
 (segment (start 141.3574 99.0601) (end 149.4726 99.0601) (width 0.3048) (layer B.Cu) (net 13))
 (segment (start 140.0875 100.33) (end 141.3574 99.0601) (width 0.3048) (layer B.Cu) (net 13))
 (segment (start 138.43 100.33) (end 140.0875 100.33) (width 0.3048) (layer B.Cu) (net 13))
 (segment (start 152.4 100.33) (end 150.7425 100.33) (width 0.3048) (layer B.Cu) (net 13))
 (segment (start 136.7287 102.0313) (end 138.43 100.33) (width 0.3048) (layer F.Cu) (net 13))
 (segment (start 136.7287 108.768) (end 136.7287 102.0313) (width 0.3048) (layer F.Cu) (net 13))
 (segment (start 137.7776 109.8169) (end 136.7287 108.768) (width 0.3048) (layer F.Cu) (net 13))
 (segment (start 137.7776 114.3533) (end 137.7776 109.8169) (width 0.3048) (layer F.Cu) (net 13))
 (segment (start 136.7725 115.3584) (end 137.7776 114.3533) (width 0.3048) (layer F.Cu) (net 13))
 (segment (start 136.7725 127) (end 136.7725 115.3584) (width 0.3048) (layer F.Cu) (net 13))
 (segment (start 138.43 127) (end 136.7725 127) (width 0.3048) (layer F.Cu) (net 13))
 (segment (start 132.4675 88.5323) (end 132.4675 92.71) (width 0.3048) (layer F.Cu) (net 14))
 (segment (start 137.1875 83.8123) (end 132.4675 88.5323) (width 0.3048) (layer F.Cu) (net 14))
 (segment (start 140.7941 83.8123) (end 137.1875 83.8123) (width 0.3048) (layer F.Cu) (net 14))
 (segment (start 143.3294 86.3476) (end 140.7941 83.8123) (width 0.3048) (layer F.Cu) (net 14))
 (segment (start 145.6783 86.3476) (end 143.3294 86.3476) (width 0.3048) (layer F.Cu) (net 14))
 (segment (start 146.4375 87.1068) (end 145.6783 86.3476) (width 0.3048) (layer F.Cu) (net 14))
 (segment (start 146.4375 92.71) (end 146.4375 87.1068) (width 0.3048) (layer F.Cu) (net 14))
 (segment (start 144.78 92.71) (end 146.4375 92.71) (width 0.3048) (layer F.Cu) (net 14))
 (segment (start 130.81 92.71) (end 132.4675 92.71) (width 0.3048) (layer F.Cu) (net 14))
 (segment (start 133.7375 93.98) (end 132.4675 95.25) (width 0.3048) (layer B.Cu) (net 16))
 (segment (start 141.8525 93.98) (end 133.7375 93.98) (width 0.3048) (layer B.Cu) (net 16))
 (segment (start 143.1225 95.25) (end 141.8525 93.98) (width 0.3048) (layer B.Cu) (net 16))
 (segment (start 144.78 95.25) (end 143.1225 95.25) (width 0.3048) (layer B.Cu) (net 16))
 (segment (start 130.81 95.25) (end 132.4675 95.25) (width 0.3048) (layer B.Cu) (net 16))
 (segment (start 133.7374 96.5201) (end 132.4675 97.79) (width 0.3048) (layer B.Cu) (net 18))
 (segment (start 141.8526 96.5201) (end 133.7374 96.5201) (width 0.3048) (layer B.Cu) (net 18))
 (segment (start 143.1225 97.79) (end 141.8526 96.5201) (width 0.3048) (layer B.Cu) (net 18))
 (segment (start 144.78 97.79) (end 143.1225 97.79) (width 0.3048) (layer B.Cu) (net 18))
 (segment (start 130.81 97.79) (end 132.4675 97.79) (width 0.3048) (layer B.Cu) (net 18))
 (segment (start 142.2598 92.71) (end 138.43 92.71) (width 0.3048) (layer B.Cu) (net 19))
 (segment (start 143.5422 91.4276) (end 142.2598 92.71) (width 0.3048) (layer B.Cu) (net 19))
 (segment (start 149.4601 91.4276) (end 143.5422 91.4276) (width 0.3048) (layer B.Cu) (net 19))
 (segment (start 150.7425 92.71) (end 149.4601 91.4276) (width 0.3048) (layer B.Cu) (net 19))
 (segment (start 152.4 92.71) (end 150.7425 92.71) (width 0.3048) (layer B.Cu) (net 19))
 (segment (start 133.7251 101.5876) (end 132.4675 100.33) (width 0.3048) (layer B.Cu) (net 20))
 (segment (start 141.8649 101.5876) (end 133.7251 101.5876) (width 0.3048) (layer B.Cu) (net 20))
 (segment (start 143.1225 100.33) (end 141.8649 101.5876) (width 0.3048) (layer B.Cu) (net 20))
 (segment (start 144.78 100.33) (end 143.1225 100.33) (width 0.3048) (layer B.Cu) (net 20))
 (segment (start 130.81 100.33) (end 132.4675 100.33) (width 0.3048) (layer B.Cu) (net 20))
 (segment (start 141.3575 88.9) (end 140.0875 90.17) (width 0.3048) (layer B.Cu) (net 21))
 (segment (start 149.4725 88.9) (end 141.3575 88.9) (width 0.3048) (layer B.Cu) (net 21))
 (segment (start 150.7425 90.17) (end 149.4725 88.9) (width 0.3048) (layer B.Cu) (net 21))
 (segment (start 152.4 90.17) (end 150.7425 90.17) (width 0.3048) (layer B.Cu) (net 21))
 (segment (start 138.43 90.17) (end 140.0875 90.17) (width 0.3048) (layer B.Cu) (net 21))
 (segment (start 133.7498 104.1523) (end 132.4675 102.87) (width 0.3048) (layer B.Cu) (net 22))
 (segment (start 141.8402 104.1523) (end 133.7498 104.1523) (width 0.3048) (layer B.Cu) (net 22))
 (segment (start 143.1225 102.87) (end 141.8402 104.1523) (width 0.3048) (layer B.Cu) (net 22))
 (segment (start 144.78 102.87) (end 143.1225 102.87) (width 0.3048) (layer B.Cu) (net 22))
 (segment (start 130.81 102.87) (end 132.4675 102.87) (width 0.3048) (layer B.Cu) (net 22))
 (segment (start 141.3698 86.3477) (end 140.0875 87.63) (width 0.3048) (layer B.Cu) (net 23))
 (segment (start 149.4602 86.3477) (end 141.3698 86.3477) (width 0.3048) (layer B.Cu) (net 23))
 (segment (start 150.7425 87.63) (end 149.4602 86.3477) (width 0.3048) (layer B.Cu) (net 23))
 (segment (start 152.4 87.63) (end 150.7425 87.63) (width 0.3048) (layer B.Cu) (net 23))
 (segment (start 138.43 87.63) (end 140.0875 87.63) (width 0.3048) (layer B.Cu) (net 23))
 (segment (start 143.1225 95.3003) (end 143.1225 87.63) (width 0.3048) (layer F.Cu) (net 24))
 (segment (start 139.3628 99.06) (end 143.1225 95.3003) (width 0.3048) (layer F.Cu) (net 24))
 (segment (start 137.5104 99.06) (end 139.3628 99.06) (width 0.3048) (layer F.Cu) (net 24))
 (segment (start 136.1117 100.4587) (end 137.5104 99.06) (width 0.3048) (layer F.Cu) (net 24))
 (segment (start 136.1117 110.1904) (end 136.1117 100.4587) (width 0.3048) (layer F.Cu) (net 24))
 (segment (start 137.1676 111.2463) (end 136.1117 110.1904) (width 0.3048) (layer F.Cu) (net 24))
 (segment (start 137.1676 113.4859) (end 137.1676 111.2463) (width 0.3048) (layer F.Cu) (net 24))
 (segment (start 134.3227 116.3308) (end 137.1676 113.4859) (width 0.3048) (layer F.Cu) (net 24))
 (segment (start 134.3227 127.6848) (end 134.3227 116.3308) (width 0.3048) (layer F.Cu) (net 24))
 (segment (start 132.4675 129.54) (end 134.3227 127.6848) (width 0.3048) (layer F.Cu) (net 24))
 (segment (start 130.81 129.54) (end 132.4675 129.54) (width 0.3048) (layer F.Cu) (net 24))
 (segment (start 144.78 87.63) (end 143.1225 87.63) (width 0.3048) (layer F.Cu) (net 24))
 (segment (start 138.43 137.16) (end 136.7725 137.16) (width 0.3048) (layer B.Cu) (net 25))
 (segment (start 138.43 129.54) (end 140.0875 129.54) (width 0.3048) (layer B.Cu) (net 25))
 (segment (start 152.4 97.79) (end 154.0575 97.79) (width 0.3048) (layer B.Cu) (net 25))
 (segment (start 154.0575 115.57) (end 140.0875 129.54) (width 0.3048) (layer B.Cu) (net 25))
 (segment (start 154.0575 97.79) (end 154.0575 115.57) (width 0.3048) (layer B.Cu) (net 25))
 (segment (start 130.81 132.08) (end 132.315 132.08) (width 0.3048) (layer B.Cu) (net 25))
 (segment (start 138.43 129.54) (end 136.7725 129.54) (width 0.3048) (layer B.Cu) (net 25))
 (segment (start 134.2325 134.62) (end 136.7725 137.16) (width 0.3048) (layer B.Cu) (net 25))
 (segment (start 134.2325 132.08) (end 134.2325 134.62) (width 0.3048) (layer B.Cu) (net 25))
 (segment (start 132.315 132.08) (end 134.2325 132.08) (width 0.3048) (layer B.Cu) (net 25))
 (segment (start 134.2325 132.08) (end 136.7725 129.54) (width 0.3048) (layer B.Cu) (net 25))
 (segment (start 130.81 124.46) (end 132.4675 124.46) (width 0.3048) (layer B.Cu) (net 25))
 (segment (start 132.4675 125.235) (end 132.4675 124.46) (width 0.3048) (layer B.Cu) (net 25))
 (segment (start 136.7725 129.54) (end 132.4675 125.235) (width 0.3048) (layer B.Cu) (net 25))
 (segment (start 154.7146 95.9071) (end 154.0575 95.25) (width 0.3048) (layer B.Cu) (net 26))
 (segment (start 154.7146 118.7452) (end 154.7146 95.9071) (width 0.3048) (layer B.Cu) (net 26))
 (segment (start 145.2774 128.1824) (end 154.7146 118.7452) (width 0.3048) (layer B.Cu) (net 26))
 (segment (start 143.8815 128.1824) (end 145.2774 128.1824) (width 0.3048) (layer B.Cu) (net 26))
 (segment (start 140.0875 131.9764) (end 143.8815 128.1824) (width 0.3048) (layer B.Cu) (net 26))
 (segment (start 140.0875 132.08) (end 140.0875 131.9764) (width 0.3048) (layer B.Cu) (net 26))
 (segment (start 138.43 132.08) (end 140.0875 132.08) (width 0.3048) (layer B.Cu) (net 26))
 (segment (start 152.4 95.25) (end 154.0575 95.25) (width 0.3048) (layer B.Cu) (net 26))
 (segment (start 132.4675 121.92) (end 132.4675 119.38) (width 0.3048) (layer F.Cu) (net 27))
 (segment (start 130.81 121.92) (end 132.4675 121.92) (width 0.3048) (layer F.Cu) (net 27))
 (segment (start 130.81 119.38) (end 132.4675 119.38) (width 0.3048) (layer F.Cu) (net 27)))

